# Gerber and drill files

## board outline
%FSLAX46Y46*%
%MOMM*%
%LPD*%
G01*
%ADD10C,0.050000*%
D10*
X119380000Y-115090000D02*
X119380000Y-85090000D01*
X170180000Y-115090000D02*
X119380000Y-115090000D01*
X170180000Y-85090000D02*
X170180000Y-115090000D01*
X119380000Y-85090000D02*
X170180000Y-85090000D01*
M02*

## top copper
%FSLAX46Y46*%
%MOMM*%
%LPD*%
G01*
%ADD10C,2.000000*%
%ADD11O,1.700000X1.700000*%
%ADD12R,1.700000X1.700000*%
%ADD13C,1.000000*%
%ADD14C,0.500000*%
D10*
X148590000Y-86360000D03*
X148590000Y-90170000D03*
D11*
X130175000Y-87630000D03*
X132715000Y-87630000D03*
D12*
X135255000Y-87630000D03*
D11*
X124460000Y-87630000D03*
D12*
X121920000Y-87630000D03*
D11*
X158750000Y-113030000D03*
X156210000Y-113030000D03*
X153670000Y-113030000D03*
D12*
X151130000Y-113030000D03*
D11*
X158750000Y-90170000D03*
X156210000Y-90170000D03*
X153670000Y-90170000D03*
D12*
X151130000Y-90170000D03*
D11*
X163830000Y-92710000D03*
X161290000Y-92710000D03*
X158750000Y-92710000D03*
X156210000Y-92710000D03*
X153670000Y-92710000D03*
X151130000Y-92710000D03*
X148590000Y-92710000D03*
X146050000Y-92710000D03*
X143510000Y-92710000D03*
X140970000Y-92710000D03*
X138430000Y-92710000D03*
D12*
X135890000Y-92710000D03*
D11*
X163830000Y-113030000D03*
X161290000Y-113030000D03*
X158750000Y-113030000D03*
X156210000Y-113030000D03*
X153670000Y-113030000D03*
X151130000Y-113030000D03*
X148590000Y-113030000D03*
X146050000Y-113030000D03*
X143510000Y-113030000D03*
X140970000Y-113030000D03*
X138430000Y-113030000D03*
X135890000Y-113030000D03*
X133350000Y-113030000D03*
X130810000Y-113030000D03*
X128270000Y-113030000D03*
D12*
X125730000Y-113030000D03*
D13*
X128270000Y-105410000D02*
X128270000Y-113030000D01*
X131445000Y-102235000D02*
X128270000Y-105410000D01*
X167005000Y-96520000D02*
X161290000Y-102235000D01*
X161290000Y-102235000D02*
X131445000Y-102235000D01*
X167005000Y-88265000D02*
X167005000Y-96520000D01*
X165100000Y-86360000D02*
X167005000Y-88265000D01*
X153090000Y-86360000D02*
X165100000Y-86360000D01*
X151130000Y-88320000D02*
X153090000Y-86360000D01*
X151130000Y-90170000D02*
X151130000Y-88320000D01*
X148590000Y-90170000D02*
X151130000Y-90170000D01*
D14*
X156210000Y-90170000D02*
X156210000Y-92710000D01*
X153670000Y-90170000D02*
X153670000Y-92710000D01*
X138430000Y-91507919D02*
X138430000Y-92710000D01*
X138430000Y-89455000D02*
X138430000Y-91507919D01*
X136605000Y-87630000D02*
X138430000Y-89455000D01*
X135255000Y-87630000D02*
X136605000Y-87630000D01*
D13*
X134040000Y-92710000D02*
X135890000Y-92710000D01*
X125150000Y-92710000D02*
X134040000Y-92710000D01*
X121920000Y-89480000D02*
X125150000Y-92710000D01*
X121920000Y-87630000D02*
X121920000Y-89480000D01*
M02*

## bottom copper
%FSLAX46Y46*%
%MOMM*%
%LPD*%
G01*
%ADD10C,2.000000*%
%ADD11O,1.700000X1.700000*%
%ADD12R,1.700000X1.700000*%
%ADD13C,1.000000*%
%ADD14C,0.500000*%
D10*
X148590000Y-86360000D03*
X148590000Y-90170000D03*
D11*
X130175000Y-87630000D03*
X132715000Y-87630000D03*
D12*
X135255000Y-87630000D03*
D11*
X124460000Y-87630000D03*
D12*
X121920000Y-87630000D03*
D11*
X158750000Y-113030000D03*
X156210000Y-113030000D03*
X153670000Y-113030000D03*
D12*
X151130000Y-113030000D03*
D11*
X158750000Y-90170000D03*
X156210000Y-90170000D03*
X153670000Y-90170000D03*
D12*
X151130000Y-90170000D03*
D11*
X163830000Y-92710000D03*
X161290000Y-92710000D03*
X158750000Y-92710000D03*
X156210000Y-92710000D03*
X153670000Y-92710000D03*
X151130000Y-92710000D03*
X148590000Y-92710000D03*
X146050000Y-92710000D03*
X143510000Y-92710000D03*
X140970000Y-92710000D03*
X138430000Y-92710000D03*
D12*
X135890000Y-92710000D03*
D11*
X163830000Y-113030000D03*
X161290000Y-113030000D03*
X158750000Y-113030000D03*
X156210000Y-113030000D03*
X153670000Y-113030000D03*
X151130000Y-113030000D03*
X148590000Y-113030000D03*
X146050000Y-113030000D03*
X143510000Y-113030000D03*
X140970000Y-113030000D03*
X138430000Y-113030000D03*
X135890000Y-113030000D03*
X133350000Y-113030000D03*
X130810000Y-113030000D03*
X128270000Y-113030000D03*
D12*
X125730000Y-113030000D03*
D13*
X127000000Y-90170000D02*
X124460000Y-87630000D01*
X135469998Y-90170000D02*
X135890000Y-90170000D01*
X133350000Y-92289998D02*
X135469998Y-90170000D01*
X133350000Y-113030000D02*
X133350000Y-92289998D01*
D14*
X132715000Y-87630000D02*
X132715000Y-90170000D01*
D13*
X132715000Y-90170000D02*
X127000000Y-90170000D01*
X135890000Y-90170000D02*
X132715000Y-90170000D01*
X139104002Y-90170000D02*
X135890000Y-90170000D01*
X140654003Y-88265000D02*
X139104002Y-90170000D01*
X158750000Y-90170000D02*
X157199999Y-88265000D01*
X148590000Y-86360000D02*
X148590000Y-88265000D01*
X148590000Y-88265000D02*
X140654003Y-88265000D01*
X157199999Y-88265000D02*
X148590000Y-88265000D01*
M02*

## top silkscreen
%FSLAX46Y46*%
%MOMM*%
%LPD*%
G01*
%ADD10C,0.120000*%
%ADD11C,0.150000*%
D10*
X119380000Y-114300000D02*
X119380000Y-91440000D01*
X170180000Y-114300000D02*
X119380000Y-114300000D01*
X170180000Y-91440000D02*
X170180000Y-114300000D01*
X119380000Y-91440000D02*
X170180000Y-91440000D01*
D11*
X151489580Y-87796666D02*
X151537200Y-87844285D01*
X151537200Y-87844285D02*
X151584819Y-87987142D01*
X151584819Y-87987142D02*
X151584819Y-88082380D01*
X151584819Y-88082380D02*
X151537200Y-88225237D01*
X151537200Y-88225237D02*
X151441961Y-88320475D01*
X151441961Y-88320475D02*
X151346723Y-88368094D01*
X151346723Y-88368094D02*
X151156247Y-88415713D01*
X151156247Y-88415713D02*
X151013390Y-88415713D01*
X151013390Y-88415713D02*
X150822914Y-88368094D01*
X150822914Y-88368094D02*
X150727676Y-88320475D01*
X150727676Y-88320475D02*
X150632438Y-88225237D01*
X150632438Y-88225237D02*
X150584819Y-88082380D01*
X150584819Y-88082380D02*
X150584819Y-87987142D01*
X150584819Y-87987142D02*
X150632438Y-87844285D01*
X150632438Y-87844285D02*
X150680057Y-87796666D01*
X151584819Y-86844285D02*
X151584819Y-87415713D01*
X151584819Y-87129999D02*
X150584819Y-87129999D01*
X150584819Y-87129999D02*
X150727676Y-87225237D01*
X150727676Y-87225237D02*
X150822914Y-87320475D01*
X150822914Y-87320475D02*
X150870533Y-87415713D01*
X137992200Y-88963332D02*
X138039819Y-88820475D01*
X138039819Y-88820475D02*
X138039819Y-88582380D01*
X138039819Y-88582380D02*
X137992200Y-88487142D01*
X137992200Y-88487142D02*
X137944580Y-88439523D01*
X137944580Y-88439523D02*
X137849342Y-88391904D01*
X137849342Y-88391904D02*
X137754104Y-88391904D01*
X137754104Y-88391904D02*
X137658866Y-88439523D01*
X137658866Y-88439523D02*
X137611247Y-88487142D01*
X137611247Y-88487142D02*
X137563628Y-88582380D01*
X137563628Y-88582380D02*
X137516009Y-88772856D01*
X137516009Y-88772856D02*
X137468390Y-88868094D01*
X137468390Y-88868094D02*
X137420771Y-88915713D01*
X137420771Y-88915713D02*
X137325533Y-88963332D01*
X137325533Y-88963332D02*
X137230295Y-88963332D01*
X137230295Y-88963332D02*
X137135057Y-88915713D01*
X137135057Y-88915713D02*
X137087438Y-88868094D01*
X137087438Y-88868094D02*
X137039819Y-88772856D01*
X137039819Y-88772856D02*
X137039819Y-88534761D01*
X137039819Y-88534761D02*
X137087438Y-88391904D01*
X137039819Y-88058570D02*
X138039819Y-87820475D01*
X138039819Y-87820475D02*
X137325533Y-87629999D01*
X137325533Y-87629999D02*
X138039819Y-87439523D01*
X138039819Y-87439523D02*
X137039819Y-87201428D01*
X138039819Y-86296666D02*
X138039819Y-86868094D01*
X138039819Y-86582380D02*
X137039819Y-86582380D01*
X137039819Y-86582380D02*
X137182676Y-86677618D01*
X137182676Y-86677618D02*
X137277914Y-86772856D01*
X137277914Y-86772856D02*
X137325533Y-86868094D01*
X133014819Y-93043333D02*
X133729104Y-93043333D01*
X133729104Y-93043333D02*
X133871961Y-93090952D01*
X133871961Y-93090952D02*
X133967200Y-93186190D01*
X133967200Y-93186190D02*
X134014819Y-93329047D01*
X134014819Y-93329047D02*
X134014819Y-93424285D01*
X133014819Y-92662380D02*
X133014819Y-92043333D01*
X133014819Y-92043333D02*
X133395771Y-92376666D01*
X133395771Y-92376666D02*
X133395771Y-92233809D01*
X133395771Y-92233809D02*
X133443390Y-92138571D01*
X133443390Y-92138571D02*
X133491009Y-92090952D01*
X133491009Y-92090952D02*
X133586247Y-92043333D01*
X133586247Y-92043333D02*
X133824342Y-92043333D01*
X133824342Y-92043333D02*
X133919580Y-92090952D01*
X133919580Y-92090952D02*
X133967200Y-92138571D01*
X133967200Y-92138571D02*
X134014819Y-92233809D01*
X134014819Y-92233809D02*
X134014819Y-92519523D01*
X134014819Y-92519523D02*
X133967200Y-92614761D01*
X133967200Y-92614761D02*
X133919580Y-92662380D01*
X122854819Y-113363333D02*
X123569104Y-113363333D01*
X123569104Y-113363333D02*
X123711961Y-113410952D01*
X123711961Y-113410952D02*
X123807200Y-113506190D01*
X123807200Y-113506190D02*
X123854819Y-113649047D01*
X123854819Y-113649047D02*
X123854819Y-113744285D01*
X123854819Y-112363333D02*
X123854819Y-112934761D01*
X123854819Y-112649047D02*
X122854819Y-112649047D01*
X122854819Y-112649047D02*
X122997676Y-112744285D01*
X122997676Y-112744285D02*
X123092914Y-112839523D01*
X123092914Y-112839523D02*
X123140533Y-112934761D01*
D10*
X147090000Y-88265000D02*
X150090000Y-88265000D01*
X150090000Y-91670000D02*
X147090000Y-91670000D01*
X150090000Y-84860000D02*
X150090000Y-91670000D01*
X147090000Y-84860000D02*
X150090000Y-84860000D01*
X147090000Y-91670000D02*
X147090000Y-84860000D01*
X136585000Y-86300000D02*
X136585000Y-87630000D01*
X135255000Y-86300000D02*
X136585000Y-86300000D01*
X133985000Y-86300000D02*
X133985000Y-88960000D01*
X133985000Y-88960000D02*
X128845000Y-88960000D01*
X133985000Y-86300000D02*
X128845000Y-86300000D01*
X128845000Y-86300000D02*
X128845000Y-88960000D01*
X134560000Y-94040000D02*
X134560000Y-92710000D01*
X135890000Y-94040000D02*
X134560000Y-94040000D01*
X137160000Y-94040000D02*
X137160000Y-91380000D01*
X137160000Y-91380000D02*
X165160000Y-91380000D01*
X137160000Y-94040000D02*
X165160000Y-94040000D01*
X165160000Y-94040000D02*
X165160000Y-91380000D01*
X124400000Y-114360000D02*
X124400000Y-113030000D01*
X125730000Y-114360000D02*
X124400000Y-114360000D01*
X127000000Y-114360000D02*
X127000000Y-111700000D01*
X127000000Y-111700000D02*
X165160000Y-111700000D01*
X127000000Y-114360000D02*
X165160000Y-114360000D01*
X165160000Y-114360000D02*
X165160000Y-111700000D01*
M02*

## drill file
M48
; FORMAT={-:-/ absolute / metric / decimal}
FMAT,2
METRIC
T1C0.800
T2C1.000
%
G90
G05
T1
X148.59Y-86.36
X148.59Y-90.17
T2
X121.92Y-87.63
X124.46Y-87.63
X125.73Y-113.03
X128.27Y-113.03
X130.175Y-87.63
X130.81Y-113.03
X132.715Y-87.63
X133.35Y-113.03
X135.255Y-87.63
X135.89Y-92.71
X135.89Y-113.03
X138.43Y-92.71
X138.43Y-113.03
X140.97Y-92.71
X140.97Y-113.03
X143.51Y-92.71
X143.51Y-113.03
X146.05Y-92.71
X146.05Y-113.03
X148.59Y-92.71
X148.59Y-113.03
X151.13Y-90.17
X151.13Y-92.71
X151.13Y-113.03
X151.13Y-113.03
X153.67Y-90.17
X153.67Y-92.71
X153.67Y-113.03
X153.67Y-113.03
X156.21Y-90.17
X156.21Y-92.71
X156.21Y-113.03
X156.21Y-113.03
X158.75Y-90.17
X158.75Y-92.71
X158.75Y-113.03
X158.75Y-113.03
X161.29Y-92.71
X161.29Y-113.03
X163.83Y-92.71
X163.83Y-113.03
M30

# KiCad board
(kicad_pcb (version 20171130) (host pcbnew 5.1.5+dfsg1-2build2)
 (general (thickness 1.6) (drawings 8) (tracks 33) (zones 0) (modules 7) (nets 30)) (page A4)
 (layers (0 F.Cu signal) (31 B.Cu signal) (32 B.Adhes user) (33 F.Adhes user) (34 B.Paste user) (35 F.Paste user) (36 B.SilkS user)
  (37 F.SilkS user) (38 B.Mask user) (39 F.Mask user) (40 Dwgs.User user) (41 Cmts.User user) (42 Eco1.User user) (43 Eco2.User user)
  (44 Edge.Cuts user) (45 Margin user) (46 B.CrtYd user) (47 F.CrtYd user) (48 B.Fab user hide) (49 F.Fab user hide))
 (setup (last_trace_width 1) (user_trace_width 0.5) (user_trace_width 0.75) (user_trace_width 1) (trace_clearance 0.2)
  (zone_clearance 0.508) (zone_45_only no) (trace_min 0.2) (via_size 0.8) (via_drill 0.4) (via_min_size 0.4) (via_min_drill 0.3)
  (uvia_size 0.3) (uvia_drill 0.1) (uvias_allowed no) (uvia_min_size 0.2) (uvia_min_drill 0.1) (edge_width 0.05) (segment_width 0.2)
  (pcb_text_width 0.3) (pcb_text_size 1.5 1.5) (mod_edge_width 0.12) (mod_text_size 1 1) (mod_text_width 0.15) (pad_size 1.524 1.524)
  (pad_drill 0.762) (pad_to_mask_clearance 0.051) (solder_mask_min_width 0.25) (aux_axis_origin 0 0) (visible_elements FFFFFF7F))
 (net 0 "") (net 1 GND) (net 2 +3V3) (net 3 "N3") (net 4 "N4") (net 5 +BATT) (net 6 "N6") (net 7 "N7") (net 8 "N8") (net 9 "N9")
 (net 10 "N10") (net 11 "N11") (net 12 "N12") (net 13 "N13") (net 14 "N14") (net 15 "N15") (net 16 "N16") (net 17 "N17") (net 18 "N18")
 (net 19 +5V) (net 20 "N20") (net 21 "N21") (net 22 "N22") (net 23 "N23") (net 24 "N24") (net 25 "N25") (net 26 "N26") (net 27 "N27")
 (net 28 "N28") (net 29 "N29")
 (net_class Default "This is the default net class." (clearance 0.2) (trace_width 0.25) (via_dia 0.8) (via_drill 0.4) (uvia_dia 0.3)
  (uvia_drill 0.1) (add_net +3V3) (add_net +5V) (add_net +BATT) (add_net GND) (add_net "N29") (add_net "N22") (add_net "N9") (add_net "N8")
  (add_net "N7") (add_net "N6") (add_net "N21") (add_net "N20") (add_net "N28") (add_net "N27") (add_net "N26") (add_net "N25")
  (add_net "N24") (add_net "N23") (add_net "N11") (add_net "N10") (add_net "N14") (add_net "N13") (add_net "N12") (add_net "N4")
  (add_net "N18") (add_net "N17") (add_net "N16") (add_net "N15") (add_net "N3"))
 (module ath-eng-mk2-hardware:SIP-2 (layer F.Cu) (at 148.59 88.265 90)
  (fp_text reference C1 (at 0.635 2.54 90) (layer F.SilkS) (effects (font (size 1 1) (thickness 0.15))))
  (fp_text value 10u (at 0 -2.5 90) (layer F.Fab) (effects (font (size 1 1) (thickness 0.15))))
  (fp_line (start 0 -1.5) (end 0 1.5) (layer F.SilkS) (width 0.12))
  (fp_line (start -3.405 1.5) (end -3.405 -1.5) (layer F.SilkS) (width 0.12))
  (fp_line (start 3.405 1.5) (end -3.405 1.5) (layer F.SilkS) (width 0.12))
  (fp_line (start 3.405 -1.5) (end 3.405 1.5) (layer F.SilkS) (width 0.12))
  (fp_line (start -3.405 -1.5) (end 3.405 -1.5) (layer F.SilkS) (width 0.12))
  (pad 2 thru_hole circle (at 1.905 0 90) (size 2 2) (drill 0.8) (layers *.Cu *.Mask) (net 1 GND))
  (pad 1 thru_hole circle (at -1.905 0 90) (size 2 2) (drill 0.8) (layers *.Cu *.Mask) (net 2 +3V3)))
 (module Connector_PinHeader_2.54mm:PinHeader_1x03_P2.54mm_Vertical (layer F.Cu) (at 135.255 87.63 270)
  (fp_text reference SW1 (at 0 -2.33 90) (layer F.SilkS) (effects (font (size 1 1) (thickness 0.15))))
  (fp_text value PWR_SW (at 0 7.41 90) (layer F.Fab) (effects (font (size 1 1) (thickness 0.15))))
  (fp_line (start -1.33 -1.33) (end 0 -1.33) (layer F.SilkS) (width 0.12))
  (fp_line (start -1.33 0) (end -1.33 -1.33) (layer F.SilkS) (width 0.12))
  (fp_line (start -1.33 1.27) (end 1.33 1.27) (layer F.SilkS) (width 0.12))
  (fp_line (start 1.33 1.27) (end 1.33 6.41) (layer F.SilkS) (width 0.12))
  (fp_line (start -1.33 1.27) (end -1.33 6.41) (layer F.SilkS) (width 0.12))
  (fp_line (start -1.33 6.41) (end 1.33 6.41) (layer F.SilkS) (width 0.12))
  (pad 3 thru_hole oval (at 0 5.08 270) (size 1.7 1.7) (drill 1) (layers *.Cu *.Mask) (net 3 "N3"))
  (pad 2 thru_hole oval (at 0 2.54 270) (size 1.7 1.7) (drill 1) (layers *.Cu *.Mask) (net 1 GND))
  (pad 1 thru_hole rect (at 0 0 270) (size 1.7 1.7) (drill 1) (layers *.Cu *.Mask) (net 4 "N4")))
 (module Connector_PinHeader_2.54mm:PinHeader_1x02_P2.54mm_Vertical (layer B.Cu) (at 121.92 87.63 270)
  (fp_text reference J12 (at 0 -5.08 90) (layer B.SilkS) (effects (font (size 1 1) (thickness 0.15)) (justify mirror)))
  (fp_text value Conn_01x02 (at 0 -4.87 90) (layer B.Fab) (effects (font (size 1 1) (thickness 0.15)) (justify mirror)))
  (pad 2 thru_hole oval (at 0 -2.54 270) (size 1.7 1.7) (drill 1) (layers *.Cu *.Mask) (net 1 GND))
  (pad 1 thru_hole rect (at 0 0 270) (size 1.7 1.7) (drill 1) (layers *.Cu *.Mask) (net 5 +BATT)))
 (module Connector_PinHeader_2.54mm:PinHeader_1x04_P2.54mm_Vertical (layer B.Cu) (at 151.13 113.03 270)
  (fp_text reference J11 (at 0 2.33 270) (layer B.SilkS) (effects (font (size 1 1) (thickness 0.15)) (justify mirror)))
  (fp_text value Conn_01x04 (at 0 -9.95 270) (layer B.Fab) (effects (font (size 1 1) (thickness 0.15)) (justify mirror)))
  (pad 4 thru_hole oval (at 0 -7.62 270) (size 1.7 1.7) (drill 1) (layers *.Cu *.Mask) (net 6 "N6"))
  (pad 3 thru_hole oval (at 0 -5.08 270) (size 1.7 1.7) (drill 1) (layers *.Cu *.Mask) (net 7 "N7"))
  (pad 2 thru_hole oval (at 0 -2.54 270) (size 1.7 1.7) (drill 1) (layers *.Cu *.Mask) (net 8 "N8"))
  (pad 1 thru_hole rect (at 0 0 270) (size 1.7 1.7) (drill 1) (layers *.Cu *.Mask) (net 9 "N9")))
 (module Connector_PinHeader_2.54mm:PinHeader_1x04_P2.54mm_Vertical (layer B.Cu) (at 151.13 90.17 270)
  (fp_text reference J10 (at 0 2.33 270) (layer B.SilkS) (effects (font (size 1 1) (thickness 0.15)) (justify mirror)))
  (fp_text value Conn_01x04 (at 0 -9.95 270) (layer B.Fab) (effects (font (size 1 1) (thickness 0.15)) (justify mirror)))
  (pad 4 thru_hole oval (at 0 -7.62 270) (size 1.7 1.7) (drill 1) (layers *.Cu *.Mask) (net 1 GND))
  (pad 3 thru_hole oval (at 0 -5.08 270) (size 1.7 1.7) (drill 1) (layers *.Cu *.Mask) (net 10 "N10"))
  (pad 2 thru_hole oval (at 0 -2.54 270) (size 1.7 1.7) (drill 1) (layers *.Cu *.Mask) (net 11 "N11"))
  (pad 1 thru_hole rect (at 0 0 270) (size 1.7 1.7) (drill 1) (layers *.Cu *.Mask) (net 2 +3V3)))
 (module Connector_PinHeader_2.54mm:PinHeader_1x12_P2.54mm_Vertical (layer F.Cu) (at 135.89 92.71 90)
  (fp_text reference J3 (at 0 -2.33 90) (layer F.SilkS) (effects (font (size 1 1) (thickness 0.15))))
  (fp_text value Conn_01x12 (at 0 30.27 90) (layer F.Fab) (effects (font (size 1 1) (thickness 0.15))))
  (fp_line (start -1.33 -1.33) (end 0 -1.33) (layer F.SilkS) (width 0.12))
  (fp_line (start -1.33 0) (end -1.33 -1.33) (layer F.SilkS) (width 0.12))
  (fp_line (start -1.33 1.27) (end 1.33 1.27) (layer F.SilkS) (width 0.12))
  (fp_line (start 1.33 1.27) (end 1.33 29.27) (layer F.SilkS) (width 0.12))
  (fp_line (start -1.33 1.27) (end -1.33 29.27) (layer F.SilkS) (width 0.12))
  (fp_line (start -1.33 29.27) (end 1.33 29.27) (layer F.SilkS) (width 0.12))
  (pad 12 thru_hole oval (at 0 27.94 90) (size 1.7 1.7) (drill 1) (layers *.Cu *.Mask) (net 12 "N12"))
  (pad 11 thru_hole oval (at 0 25.4 90) (size 1.7 1.7) (drill 1) (layers *.Cu *.Mask) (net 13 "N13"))
  (pad 10 thru_hole oval (at 0 22.86 90) (size 1.7 1.7) (drill 1) (layers *.Cu *.Mask) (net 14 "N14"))
  (pad 9 thru_hole oval (at 0 20.32 90) (size 1.7 1.7) (drill 1) (layers *.Cu *.Mask) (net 10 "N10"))
  (pad 8 thru_hole oval (at 0 17.78 90) (size 1.7 1.7) (drill 1) (layers *.Cu *.Mask) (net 11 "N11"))
  (pad 7 thru_hole oval (at 0 15.24 90) (size 1.7 1.7) (drill 1) (layers *.Cu *.Mask) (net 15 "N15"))
  (pad 6 thru_hole oval (at 0 12.7 90) (size 1.7 1.7) (drill 1) (layers *.Cu *.Mask) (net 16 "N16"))
  (pad 5 thru_hole oval (at 0 10.16 90) (size 1.7 1.7) (drill 1) (layers *.Cu *.Mask) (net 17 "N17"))
  (pad 4 thru_hole oval (at 0 7.62 90) (size 1.7 1.7) (drill 1) (layers *.Cu *.Mask) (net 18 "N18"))
  (pad 3 thru_hole oval (at 0 5.08 90) (size 1.7 1.7) (drill 1) (layers *.Cu *.Mask) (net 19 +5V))
  (pad 2 thru_hole oval (at 0 2.54 90) (size 1.7 1.7) (drill 1) (layers *.Cu *.Mask) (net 4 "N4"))
  (pad 1 thru_hole rect (at 0 0 90) (size 1.7 1.7) (drill 1) (layers *.Cu *.Mask) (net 5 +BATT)))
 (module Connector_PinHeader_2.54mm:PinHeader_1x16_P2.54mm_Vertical (layer F.Cu) (at 125.73 113.03 90)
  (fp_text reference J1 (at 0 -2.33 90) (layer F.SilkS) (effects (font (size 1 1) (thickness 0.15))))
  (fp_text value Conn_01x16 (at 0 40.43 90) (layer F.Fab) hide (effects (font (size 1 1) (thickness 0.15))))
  (fp_line (start -1.33 -1.33) (end 0 -1.33) (layer F.SilkS) (width 0.12))
  (fp_line (start -1.33 0) (end -1.33 -1.33) (layer F.SilkS) (width 0.12))
  (fp_line (start -1.33 1.27) (end 1.33 1.27) (layer F.SilkS) (width 0.12))
  (fp_line (start 1.33 1.27) (end 1.33 39.43) (layer F.SilkS) (width 0.12))
  (fp_line (start -1.33 1.27) (end -1.33 39.43) (layer F.SilkS) (width 0.12))
  (fp_line (start -1.33 39.43) (end 1.33 39.43) (layer F.SilkS) (width 0.12))
  (pad 16 thru_hole oval (at 0 38.1 90) (size 1.7 1.7) (drill 1) (layers *.Cu *.Mask) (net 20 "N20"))
  (pad 15 thru_hole oval (at 0 35.56 90) (size 1.7 1.7) (drill 1) (layers *.Cu *.Mask) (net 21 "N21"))
  (pad 14 thru_hole oval (at 0 33.02 90) (size 1.7 1.7) (drill 1) (layers *.Cu *.Mask) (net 6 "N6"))
  (pad 13 thru_hole oval (at 0 30.48 90) (size 1.7 1.7) (drill 1) (layers *.Cu *.Mask) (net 7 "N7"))
  (pad 12 thru_hole oval (at 0 27.94 90) (size 1.7 1.7) (drill 1) (layers *.Cu *.Mask) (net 8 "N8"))
  (pad 11 thru_hole oval (at 0 25.4 90) (size 1.7 1.7) (drill 1) (layers *.Cu *.Mask) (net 9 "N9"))
  (pad 10 thru_hole oval (at 0 22.86 90) (size 1.7 1.7) (drill 1) (layers *.Cu *.Mask) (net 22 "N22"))
  (pad 9 thru_hole oval (at 0 20.32 90) (size 1.7 1.7) (drill 1) (layers *.Cu *.Mask) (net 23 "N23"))
  (pad 8 thru_hole oval (at 0 17.78 90) (size 1.7 1.7) (drill 1) (layers *.Cu *.Mask) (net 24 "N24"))
  (pad 7 thru_hole oval (at 0 15.24 90) (size 1.7 1.7) (drill 1) (layers *.Cu *.Mask) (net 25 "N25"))
  (pad 6 thru_hole oval (at 0 12.7 90) (size 1.7 1.7) (drill 1) (layers *.Cu *.Mask) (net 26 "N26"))
  (pad 5 thru_hole oval (at 0 10.16 90) (size 1.7 1.7) (drill 1) (layers *.Cu *.Mask) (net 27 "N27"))
  (pad 4 thru_hole oval (at 0 7.62 90) (size 1.7 1.7) (drill 1) (layers *.Cu *.Mask) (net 1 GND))
  (pad 3 thru_hole oval (at 0 5.08 90) (size 1.7 1.7) (drill 1) (layers *.Cu *.Mask) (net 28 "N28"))
  (pad 2 thru_hole oval (at 0 2.54 90) (size 1.7 1.7) (drill 1) (layers *.Cu *.Mask) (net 2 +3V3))
  (pad 1 thru_hole rect (at 0 0 90) (size 1.7 1.7) (drill 1) (layers *.Cu *.Mask) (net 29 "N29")))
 (gr_line (start 119.38 114.3) (end 119.38 91.44) (layer F.SilkS) (width 0.12))
 (gr_line (start 170.18 114.3) (end 119.38 114.3) (layer F.SilkS) (width 0.12))
 (gr_line (start 170.18 91.44) (end 170.18 114.3) (layer F.SilkS) (width 0.12))
 (gr_line (start 119.38 91.44) (end 170.18 91.44) (layer F.SilkS) (width 0.12))
 (gr_line (start 119.38 115.09) (end 119.38 85.09) (layer Edge.Cuts) (width 0.05))
 (gr_line (start 170.18 115.09) (end 119.38 115.09) (layer Edge.Cuts) (width 0.05))
 (gr_line (start 170.18 85.09) (end 170.18 115.09) (layer Edge.Cuts) (width 0.05))
 (gr_line (start 119.38 85.09) (end 170.18 85.09) (layer Edge.Cuts) (width 0.05))
 (segment (start 127 90.17) (end 124.46 87.63) (width 1) (layer B.Cu) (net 1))
 (segment (start 135.469998 90.17) (end 135.89 90.17) (width 1) (layer B.Cu) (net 1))
 (segment (start 133.35 92.289998) (end 135.469998 90.17) (width 1) (layer B.Cu) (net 1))
 (segment (start 133.35 113.03) (end 133.35 92.289998) (width 1) (layer B.Cu) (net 1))
 (segment (start 132.715 87.63) (end 132.715 90.17) (width 0.5) (layer B.Cu) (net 1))
 (segment (start 132.715 90.17) (end 127 90.17) (width 1) (layer B.Cu) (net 1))
 (segment (start 135.89 90.17) (end 132.715 90.17) (width 1) (layer B.Cu) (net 1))
 (segment (start 139.104002 90.17) (end 135.89 90.17) (width 1) (layer B.Cu) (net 1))
 (segment (start 140.654003 88.265) (end 139.104002 90.17) (width 1) (layer B.Cu) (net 1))
 (segment (start 158.75 90.17) (end 157.199999 88.265) (width 1) (layer B.Cu) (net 1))
 (segment (start 148.59 86.36) (end 148.59 88.265) (width 1) (layer B.Cu) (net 1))
 (segment (start 148.59 88.265) (end 140.654003 88.265) (width 1) (layer B.Cu) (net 1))
 (segment (start 157.199999 88.265) (end 148.59 88.265) (width 1) (layer B.Cu) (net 1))
 (segment (start 128.27 105.41) (end 128.27 113.03) (width 1) (layer F.Cu) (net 2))
 (segment (start 131.445 102.235) (end 128.27 105.41) (width 1) (layer F.Cu) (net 2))
 (segment (start 167.005 96.52) (end 161.29 102.235) (width 1) (layer F.Cu) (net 2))
 (segment (start 161.29 102.235) (end 131.445 102.235) (width 1) (layer F.Cu) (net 2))
 (segment (start 167.005 88.265) (end 167.005 96.52) (width 1) (layer F.Cu) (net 2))
 (segment (start 165.1 86.36) (end 167.005 88.265) (width 1) (layer F.Cu) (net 2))
 (segment (start 153.09 86.36) (end 165.1 86.36) (width 1) (layer F.Cu) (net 2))
 (segment (start 151.13 88.32) (end 153.09 86.36) (width 1) (layer F.Cu) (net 2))
 (segment (start 151.13 90.17) (end 151.13 88.32) (width 1) (layer F.Cu) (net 2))
 (segment (start 148.59 90.17) (end 151.13 90.17) (width 1) (layer F.Cu) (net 2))
 (segment (start 156.21 90.17) (end 156.21 92.71) (width 0.5) (layer F.Cu) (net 10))
 (segment (start 153.67 90.17) (end 153.67 92.71) (width 0.5) (layer F.Cu) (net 11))
 (segment (start 138.43 91.507919) (end 138.43 92.71) (width 0.5) (layer F.Cu) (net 4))
 (segment (start 138.43 89.455) (end 138.43 91.507919) (width 0.5) (layer F.Cu) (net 4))
 (segment (start 136.605 87.63) (end 138.43 89.455) (width 0.5) (layer F.Cu) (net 4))
 (segment (start 135.255 87.63) (end 136.605 87.63) (width 0.5) (layer F.Cu) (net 4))
 (segment (start 134.04 92.71) (end 135.89 92.71) (width 1) (layer F.Cu) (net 5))
 (segment (start 125.15 92.71) (end 134.04 92.71) (width 1) (layer F.Cu) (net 5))
 (segment (start 121.92 89.48) (end 125.15 92.71) (width 1) (layer F.Cu) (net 5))
 (segment (start 121.92 87.63) (end 121.92 89.48) (width 1) (layer F.Cu) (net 5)))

